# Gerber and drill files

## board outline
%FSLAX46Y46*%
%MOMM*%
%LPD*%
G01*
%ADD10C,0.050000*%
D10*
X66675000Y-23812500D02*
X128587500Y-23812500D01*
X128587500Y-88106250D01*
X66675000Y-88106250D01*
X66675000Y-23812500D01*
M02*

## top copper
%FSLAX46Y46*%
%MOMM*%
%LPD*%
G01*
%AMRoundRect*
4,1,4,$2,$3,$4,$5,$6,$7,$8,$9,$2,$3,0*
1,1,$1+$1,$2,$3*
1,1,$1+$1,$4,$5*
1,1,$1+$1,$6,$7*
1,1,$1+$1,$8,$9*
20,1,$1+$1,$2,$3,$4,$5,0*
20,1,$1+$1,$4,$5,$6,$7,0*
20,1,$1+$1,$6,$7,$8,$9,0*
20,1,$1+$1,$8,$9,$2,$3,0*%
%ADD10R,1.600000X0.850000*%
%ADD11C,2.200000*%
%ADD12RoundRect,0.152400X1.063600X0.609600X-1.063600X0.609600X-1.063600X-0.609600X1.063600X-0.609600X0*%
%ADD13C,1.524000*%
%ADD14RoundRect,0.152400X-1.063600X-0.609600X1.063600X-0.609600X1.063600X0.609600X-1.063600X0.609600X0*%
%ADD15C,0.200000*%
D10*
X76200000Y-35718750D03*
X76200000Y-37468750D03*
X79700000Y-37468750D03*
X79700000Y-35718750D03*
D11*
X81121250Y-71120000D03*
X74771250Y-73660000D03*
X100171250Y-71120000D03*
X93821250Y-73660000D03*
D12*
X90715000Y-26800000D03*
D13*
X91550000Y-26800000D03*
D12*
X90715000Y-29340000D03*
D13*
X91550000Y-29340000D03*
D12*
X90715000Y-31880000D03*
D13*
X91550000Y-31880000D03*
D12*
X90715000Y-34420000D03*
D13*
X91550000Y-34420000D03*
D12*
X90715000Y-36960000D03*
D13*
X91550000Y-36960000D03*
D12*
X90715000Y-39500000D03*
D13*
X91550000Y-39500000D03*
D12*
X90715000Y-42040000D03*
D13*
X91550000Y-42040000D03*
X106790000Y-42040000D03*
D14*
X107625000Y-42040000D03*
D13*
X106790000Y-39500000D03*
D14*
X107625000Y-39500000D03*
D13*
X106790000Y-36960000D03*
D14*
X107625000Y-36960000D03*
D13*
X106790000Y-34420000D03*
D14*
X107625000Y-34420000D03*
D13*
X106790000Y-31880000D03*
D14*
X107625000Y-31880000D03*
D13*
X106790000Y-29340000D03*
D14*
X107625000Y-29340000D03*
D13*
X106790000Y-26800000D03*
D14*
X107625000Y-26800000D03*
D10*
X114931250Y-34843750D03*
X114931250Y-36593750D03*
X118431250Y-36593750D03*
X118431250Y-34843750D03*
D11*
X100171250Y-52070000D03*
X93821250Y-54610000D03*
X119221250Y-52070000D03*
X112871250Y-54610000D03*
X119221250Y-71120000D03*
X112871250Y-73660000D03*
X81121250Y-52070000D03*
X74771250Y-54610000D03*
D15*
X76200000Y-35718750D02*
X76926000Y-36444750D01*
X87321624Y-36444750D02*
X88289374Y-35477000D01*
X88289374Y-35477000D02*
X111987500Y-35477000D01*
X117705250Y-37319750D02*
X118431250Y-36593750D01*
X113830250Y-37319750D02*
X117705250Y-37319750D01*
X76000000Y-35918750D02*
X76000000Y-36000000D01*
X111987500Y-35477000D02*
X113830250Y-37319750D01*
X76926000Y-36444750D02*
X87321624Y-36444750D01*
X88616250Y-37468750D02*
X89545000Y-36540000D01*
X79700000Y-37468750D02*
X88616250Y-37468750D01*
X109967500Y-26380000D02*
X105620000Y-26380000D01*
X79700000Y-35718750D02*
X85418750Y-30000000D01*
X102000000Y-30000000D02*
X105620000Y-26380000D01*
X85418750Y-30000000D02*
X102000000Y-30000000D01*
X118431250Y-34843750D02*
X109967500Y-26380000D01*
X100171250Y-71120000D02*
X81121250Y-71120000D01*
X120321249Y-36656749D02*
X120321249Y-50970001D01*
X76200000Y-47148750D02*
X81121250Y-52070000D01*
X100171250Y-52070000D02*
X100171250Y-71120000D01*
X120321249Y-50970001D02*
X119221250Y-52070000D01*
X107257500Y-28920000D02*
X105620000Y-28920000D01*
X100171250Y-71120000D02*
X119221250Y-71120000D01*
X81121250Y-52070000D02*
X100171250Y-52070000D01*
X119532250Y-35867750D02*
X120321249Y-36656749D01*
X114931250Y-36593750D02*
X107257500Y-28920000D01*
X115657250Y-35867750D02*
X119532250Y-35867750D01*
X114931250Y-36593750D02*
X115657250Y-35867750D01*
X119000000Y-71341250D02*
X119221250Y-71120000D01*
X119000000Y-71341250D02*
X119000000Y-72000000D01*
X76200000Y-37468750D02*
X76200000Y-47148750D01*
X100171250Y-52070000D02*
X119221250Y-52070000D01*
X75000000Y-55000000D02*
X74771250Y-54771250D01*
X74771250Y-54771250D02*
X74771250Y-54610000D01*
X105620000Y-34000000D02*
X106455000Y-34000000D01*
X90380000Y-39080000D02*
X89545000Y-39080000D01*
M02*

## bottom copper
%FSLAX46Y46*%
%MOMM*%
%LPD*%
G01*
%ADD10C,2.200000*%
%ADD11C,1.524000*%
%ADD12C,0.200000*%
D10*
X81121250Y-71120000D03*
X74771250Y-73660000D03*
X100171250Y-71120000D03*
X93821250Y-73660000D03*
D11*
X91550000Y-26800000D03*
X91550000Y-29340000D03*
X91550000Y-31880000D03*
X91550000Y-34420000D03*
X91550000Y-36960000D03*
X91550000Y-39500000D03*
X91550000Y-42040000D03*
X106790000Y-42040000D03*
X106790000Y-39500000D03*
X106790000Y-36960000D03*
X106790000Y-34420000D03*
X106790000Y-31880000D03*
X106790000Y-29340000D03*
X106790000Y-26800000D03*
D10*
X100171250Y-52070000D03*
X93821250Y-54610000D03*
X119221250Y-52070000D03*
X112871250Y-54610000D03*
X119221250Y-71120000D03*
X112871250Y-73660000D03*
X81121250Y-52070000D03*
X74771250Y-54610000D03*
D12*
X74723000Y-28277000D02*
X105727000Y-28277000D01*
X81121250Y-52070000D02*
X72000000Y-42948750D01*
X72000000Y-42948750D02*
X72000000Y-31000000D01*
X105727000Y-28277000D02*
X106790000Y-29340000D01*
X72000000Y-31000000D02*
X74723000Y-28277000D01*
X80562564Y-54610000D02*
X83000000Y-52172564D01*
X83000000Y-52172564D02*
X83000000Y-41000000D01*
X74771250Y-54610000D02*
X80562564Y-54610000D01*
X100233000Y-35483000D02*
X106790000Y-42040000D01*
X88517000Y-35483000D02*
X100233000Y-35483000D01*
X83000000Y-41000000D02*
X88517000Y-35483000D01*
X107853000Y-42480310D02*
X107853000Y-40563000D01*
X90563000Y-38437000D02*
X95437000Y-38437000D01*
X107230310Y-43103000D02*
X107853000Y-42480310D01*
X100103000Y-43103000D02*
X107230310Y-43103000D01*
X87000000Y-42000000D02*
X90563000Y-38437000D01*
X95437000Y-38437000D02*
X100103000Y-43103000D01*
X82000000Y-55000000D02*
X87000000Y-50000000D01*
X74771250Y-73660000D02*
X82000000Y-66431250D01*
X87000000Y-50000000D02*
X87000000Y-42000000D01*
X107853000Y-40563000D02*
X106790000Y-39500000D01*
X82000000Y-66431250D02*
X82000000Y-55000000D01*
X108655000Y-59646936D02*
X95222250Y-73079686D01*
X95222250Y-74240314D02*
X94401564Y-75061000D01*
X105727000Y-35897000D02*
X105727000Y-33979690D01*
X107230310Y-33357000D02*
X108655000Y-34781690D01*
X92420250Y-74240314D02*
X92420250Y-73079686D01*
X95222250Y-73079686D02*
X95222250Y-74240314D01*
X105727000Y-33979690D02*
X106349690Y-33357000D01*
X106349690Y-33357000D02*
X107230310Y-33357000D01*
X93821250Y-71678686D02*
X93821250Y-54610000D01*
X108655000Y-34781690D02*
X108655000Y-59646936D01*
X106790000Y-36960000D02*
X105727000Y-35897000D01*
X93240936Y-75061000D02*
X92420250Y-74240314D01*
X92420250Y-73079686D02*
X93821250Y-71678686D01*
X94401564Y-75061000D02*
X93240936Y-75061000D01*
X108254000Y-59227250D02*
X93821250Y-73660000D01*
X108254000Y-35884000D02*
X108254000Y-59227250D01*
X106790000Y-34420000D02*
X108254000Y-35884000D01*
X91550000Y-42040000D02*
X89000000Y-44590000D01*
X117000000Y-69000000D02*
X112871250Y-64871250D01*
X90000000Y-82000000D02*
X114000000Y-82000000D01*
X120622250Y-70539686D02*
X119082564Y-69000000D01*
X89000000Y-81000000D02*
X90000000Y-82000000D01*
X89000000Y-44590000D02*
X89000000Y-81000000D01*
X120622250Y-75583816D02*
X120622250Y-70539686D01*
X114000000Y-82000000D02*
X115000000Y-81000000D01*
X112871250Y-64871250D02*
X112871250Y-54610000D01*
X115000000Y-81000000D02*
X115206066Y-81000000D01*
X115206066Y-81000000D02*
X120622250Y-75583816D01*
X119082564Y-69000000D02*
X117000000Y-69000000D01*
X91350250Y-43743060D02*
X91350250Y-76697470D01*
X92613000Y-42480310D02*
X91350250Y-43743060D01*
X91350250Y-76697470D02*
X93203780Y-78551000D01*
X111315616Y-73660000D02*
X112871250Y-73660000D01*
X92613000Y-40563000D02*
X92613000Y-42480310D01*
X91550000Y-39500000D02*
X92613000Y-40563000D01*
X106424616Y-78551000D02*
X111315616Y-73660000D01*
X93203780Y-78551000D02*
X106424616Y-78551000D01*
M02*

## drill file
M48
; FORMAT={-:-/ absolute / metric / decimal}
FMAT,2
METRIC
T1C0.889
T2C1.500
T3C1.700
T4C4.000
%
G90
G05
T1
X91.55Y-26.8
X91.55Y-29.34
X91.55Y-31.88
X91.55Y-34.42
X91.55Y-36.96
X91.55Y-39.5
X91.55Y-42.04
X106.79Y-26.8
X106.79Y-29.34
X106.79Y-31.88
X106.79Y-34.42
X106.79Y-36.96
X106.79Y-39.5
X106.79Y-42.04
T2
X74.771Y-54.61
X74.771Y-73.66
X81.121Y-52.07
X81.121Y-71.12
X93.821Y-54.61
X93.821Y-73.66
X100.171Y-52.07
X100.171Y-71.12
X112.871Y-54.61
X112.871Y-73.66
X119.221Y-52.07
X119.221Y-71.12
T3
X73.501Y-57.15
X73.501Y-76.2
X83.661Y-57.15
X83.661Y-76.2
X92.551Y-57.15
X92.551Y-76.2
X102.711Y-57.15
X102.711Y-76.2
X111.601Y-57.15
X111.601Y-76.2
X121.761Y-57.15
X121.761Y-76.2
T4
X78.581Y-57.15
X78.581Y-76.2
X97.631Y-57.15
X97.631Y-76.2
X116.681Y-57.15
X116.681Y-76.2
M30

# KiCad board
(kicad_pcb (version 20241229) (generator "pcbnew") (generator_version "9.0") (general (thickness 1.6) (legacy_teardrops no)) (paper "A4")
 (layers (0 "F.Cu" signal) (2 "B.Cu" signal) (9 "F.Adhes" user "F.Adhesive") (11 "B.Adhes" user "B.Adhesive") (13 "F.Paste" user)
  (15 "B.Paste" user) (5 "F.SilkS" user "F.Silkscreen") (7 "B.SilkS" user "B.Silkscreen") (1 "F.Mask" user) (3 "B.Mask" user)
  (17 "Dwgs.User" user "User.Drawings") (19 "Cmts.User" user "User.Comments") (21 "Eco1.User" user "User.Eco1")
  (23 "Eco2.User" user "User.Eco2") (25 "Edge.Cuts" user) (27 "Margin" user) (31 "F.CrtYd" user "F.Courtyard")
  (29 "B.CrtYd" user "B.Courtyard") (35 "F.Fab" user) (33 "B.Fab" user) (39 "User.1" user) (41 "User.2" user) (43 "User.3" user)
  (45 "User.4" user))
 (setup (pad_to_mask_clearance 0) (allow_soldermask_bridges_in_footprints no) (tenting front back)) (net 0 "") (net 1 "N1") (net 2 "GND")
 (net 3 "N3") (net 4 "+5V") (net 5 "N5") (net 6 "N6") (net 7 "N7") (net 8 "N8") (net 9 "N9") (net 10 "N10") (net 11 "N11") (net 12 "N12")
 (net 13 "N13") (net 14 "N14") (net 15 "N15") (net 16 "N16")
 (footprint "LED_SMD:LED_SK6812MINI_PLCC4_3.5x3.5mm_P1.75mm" (layer "F.Cu") (at 77.95 36.59375)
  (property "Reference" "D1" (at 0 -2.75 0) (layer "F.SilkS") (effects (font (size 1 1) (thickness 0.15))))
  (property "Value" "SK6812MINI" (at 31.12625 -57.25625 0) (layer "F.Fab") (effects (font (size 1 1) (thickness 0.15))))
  (pad "1" smd rect (at -1.75 -0.875) (size 1.6 0.85) (layers "F.Cu" "F.Mask" "F.Paste") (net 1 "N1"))
  (pad "2" smd rect (at -1.75 0.875) (size 1.6 0.85) (layers "F.Cu" "F.Mask" "F.Paste") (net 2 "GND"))
  (pad "3" smd rect (at 1.75 0.875) (size 1.6 0.85) (layers "F.Cu" "F.Mask" "F.Paste") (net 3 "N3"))
  (pad "4" smd rect (at 1.75 -0.875) (size 1.6 0.85) (layers "F.Cu" "F.Mask" "F.Paste") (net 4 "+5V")))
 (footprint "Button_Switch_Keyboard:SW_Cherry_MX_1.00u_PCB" (layer "F.Cu") (at 81.12125 71.12)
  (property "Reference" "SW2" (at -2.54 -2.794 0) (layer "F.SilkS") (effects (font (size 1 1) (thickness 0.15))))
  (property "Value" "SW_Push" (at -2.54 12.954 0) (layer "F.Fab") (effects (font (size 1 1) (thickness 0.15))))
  (pad "" np_thru_hole circle (at -7.62 5.08) (size 1.7 1.7) (drill 1.7) (layers "*.Cu" "*.Mask"))
  (pad "" np_thru_hole circle (at -2.54 5.08) (size 4 4) (drill 4) (layers "*.Cu" "*.Mask"))
  (pad "" np_thru_hole circle (at 2.54 5.08) (size 1.7 1.7) (drill 1.7) (layers "*.Cu" "*.Mask"))
  (pad "1" thru_hole circle (at 0 0) (size 2.2 2.2) (drill 1.5) (layers "*.Cu" "*.Mask") (remove_unused_layers no) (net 2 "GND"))
  (pad "2" thru_hole circle (at -6.35 2.54) (size 2.2 2.2) (drill 1.5) (layers "*.Cu" "*.Mask") (remove_unused_layers no) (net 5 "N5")))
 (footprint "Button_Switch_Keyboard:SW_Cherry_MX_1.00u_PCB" (layer "F.Cu") (at 100.17125 71.12)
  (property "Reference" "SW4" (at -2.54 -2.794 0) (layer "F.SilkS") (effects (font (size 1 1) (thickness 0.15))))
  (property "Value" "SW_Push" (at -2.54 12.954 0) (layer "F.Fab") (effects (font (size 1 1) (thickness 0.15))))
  (pad "" np_thru_hole circle (at -7.62 5.08) (size 1.7 1.7) (drill 1.7) (layers "*.Cu" "*.Mask"))
  (pad "" np_thru_hole circle (at -2.54 5.08) (size 4 4) (drill 4) (layers "*.Cu" "*.Mask"))
  (pad "" np_thru_hole circle (at 2.54 5.08) (size 1.7 1.7) (drill 1.7) (layers "*.Cu" "*.Mask"))
  (pad "1" thru_hole circle (at 0 0) (size 2.2 2.2) (drill 1.5) (layers "*.Cu" "*.Mask") (remove_unused_layers no) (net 2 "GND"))
  (pad "2" thru_hole circle (at -6.35 2.54) (size 2.2 2.2) (drill 1.5) (layers "*.Cu" "*.Mask") (remove_unused_layers no) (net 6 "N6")))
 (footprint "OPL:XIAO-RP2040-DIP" (layer "F.Cu") (at 99.17 34.42)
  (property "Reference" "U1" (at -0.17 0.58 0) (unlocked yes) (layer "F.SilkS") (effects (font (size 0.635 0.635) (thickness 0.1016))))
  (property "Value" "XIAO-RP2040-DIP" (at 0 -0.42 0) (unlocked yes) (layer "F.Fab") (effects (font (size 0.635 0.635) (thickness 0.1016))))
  (pad "1" smd roundrect (at -8.455 -7.62 180) (size 2.432 1.524) (layers "F.Cu" "F.Mask") (roundrect_rratio 0.1) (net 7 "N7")
   (thermal_bridge_angle 45))
  (pad "1" thru_hole circle (at -7.62 -7.62 180) (size 1.524 1.524) (drill 0.889) (layers "*.Cu" "*.Mask") (remove_unused_layers no)
   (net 7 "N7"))
  (pad "2" smd roundrect (at -8.455 -5.08 180) (size 2.432 1.524) (layers "F.Cu" "F.Mask") (roundrect_rratio 0.1) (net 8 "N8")
   (thermal_bridge_angle 45))
  (pad "2" thru_hole circle (at -7.62 -5.08 180) (size 1.524 1.524) (drill 0.889) (layers "*.Cu" "*.Mask") (remove_unused_layers no)
   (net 8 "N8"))
  (pad "3" smd roundrect (at -8.455 -2.54 180) (size 2.432 1.524) (layers "F.Cu" "F.Mask") (roundrect_rratio 0.1) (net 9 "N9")
   (thermal_bridge_angle 45))
  (pad "3" thru_hole circle (at -7.62 -2.54 180) (size 1.524 1.524) (drill 0.889) (layers "*.Cu" "*.Mask") (remove_unused_layers no)
   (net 9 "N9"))
  (pad "4" smd roundrect (at -8.455 0 180) (size 2.432 1.524) (layers "F.Cu" "F.Mask") (roundrect_rratio 0.1) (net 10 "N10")
   (thermal_bridge_angle 45))
  (pad "4" thru_hole circle (at -7.62 0 180) (size 1.524 1.524) (drill 0.889) (layers "*.Cu" "*.Mask") (remove_unused_layers no)
   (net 10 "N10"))
  (pad "5" smd roundrect (at -8.455 2.54 180) (size 2.432 1.524) (layers "F.Cu" "F.Mask") (roundrect_rratio 0.1) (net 3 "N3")
   (thermal_bridge_angle 45))
  (pad "5" thru_hole circle (at -7.62 2.54 180) (size 1.524 1.524) (drill 0.889) (layers "*.Cu" "*.Mask") (remove_unused_layers no)
   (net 3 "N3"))
  (pad "6" smd roundrect (at -8.455 5.08 180) (size 2.432 1.524) (layers "F.Cu" "F.Mask") (roundrect_rratio 0.1) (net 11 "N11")
   (thermal_bridge_angle 45))
  (pad "6" thru_hole circle (at -7.62 5.08 180) (size 1.524 1.524) (drill 0.889) (layers "*.Cu" "*.Mask") (remove_unused_layers no)
   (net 11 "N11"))
  (pad "7" smd roundrect (at -8.455 7.62 180) (size 2.432 1.524) (layers "F.Cu" "F.Mask") (roundrect_rratio 0.1) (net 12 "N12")
   (thermal_bridge_angle 45))
  (pad "7" thru_hole circle (at -7.62 7.62 180) (size 1.524 1.524) (drill 0.889) (layers "*.Cu" "*.Mask") (remove_unused_layers no)
   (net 12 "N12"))
  (pad "8" thru_hole circle (at 7.62 7.62) (size 1.524 1.524) (drill 0.889) (layers "*.Cu" "*.Mask") (remove_unused_layers no)
   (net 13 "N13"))
  (pad "8" smd roundrect (at 8.455 7.62) (size 2.432 1.524) (layers "F.Cu" "F.Mask") (roundrect_rratio 0.1) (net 13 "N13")
   (thermal_bridge_angle 45))
  (pad "9" thru_hole circle (at 7.62 5.08) (size 1.524 1.524) (drill 0.889) (layers "*.Cu" "*.Mask") (remove_unused_layers no) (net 5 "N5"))
  (pad "9" smd roundrect (at 8.455 5.08) (size 2.432 1.524) (layers "F.Cu" "F.Mask") (roundrect_rratio 0.1) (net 5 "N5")
   (thermal_bridge_angle 45))
  (pad "10" thru_hole circle (at 7.62 2.54) (size 1.524 1.524) (drill 0.889) (layers "*.Cu" "*.Mask") (remove_unused_layers no)
   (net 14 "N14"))
  (pad "10" smd roundrect (at 8.455 2.54) (size 2.432 1.524) (layers "F.Cu" "F.Mask") (roundrect_rratio 0.1) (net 14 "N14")
   (thermal_bridge_angle 45))
  (pad "11" thru_hole circle (at 7.62 0) (size 1.524 1.524) (drill 0.889) (layers "*.Cu" "*.Mask") (remove_unused_layers no) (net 6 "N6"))
  (pad "11" smd roundrect (at 8.455 0) (size 2.432 1.524) (layers "F.Cu" "F.Mask") (roundrect_rratio 0.1) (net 6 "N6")
   (thermal_bridge_angle 45))
  (pad "12" thru_hole circle (at 7.62 -2.54) (size 1.524 1.524) (drill 0.889) (layers "*.Cu" "*.Mask") (remove_unused_layers no)
   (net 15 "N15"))
  (pad "12" smd roundrect (at 8.455 -2.54) (size 2.432 1.524) (layers "F.Cu" "F.Mask") (roundrect_rratio 0.1) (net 15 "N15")
   (thermal_bridge_angle 45))
  (pad "13" thru_hole circle (at 7.62 -5.08) (size 1.524 1.524) (drill 0.889) (layers "*.Cu" "*.Mask") (remove_unused_layers no)
   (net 2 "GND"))
  (pad "13" smd roundrect (at 8.455 -5.08) (size 2.432 1.524) (layers "F.Cu" "F.Mask") (roundrect_rratio 0.1) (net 2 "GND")
   (thermal_bridge_angle 45))
  (pad "14" thru_hole circle (at 7.62 -7.62) (size 1.524 1.524) (drill 0.889) (layers "*.Cu" "*.Mask") (remove_unused_layers no)
   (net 4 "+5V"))
  (pad "14" smd roundrect (at 8.455 -7.62) (size 2.432 1.524) (layers "F.Cu" "F.Mask") (roundrect_rratio 0.1) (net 4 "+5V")
   (thermal_bridge_angle 45)))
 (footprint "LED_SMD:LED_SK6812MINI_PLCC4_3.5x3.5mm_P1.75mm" (layer "F.Cu") (at 116.68125 35.71875)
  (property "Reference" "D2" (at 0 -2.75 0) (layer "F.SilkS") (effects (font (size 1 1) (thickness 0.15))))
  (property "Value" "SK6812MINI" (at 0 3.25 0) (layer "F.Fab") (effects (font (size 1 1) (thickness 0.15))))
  (pad "1" smd rect (at -1.75 -0.875) (size 1.6 0.85) (layers "F.Cu" "F.Mask" "F.Paste") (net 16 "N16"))
  (pad "2" smd rect (at -1.75 0.875) (size 1.6 0.85) (layers "F.Cu" "F.Mask" "F.Paste") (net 2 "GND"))
  (pad "3" smd rect (at 1.75 0.875) (size 1.6 0.85) (layers "F.Cu" "F.Mask" "F.Paste") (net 1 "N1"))
  (pad "4" smd rect (at 1.75 -0.875) (size 1.6 0.85) (layers "F.Cu" "F.Mask" "F.Paste") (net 4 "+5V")))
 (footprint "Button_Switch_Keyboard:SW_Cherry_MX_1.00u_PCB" (layer "F.Cu") (at 100.17125 52.07)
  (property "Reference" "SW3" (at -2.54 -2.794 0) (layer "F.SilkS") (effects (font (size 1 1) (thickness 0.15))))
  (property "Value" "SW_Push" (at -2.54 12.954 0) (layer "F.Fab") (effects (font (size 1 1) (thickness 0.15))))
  (pad "" np_thru_hole circle (at -7.62 5.08) (size 1.7 1.7) (drill 1.7) (layers "*.Cu" "*.Mask"))
  (pad "" np_thru_hole circle (at -2.54 5.08) (size 4 4) (drill 4) (layers "*.Cu" "*.Mask"))
  (pad "" np_thru_hole circle (at 2.54 5.08) (size 1.7 1.7) (drill 1.7) (layers "*.Cu" "*.Mask"))
  (pad "1" thru_hole circle (at 0 0) (size 2.2 2.2) (drill 1.5) (layers "*.Cu" "*.Mask") (remove_unused_layers no) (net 2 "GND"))
  (pad "2" thru_hole circle (at -6.35 2.54) (size 2.2 2.2) (drill 1.5) (layers "*.Cu" "*.Mask") (remove_unused_layers no) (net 14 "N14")))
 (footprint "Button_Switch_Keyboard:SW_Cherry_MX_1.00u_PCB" (layer "F.Cu") (at 119.22125 52.07)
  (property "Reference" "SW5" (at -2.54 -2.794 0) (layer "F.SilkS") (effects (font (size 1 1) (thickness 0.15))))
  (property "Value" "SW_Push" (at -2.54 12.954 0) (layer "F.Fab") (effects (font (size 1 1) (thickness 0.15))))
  (pad "" np_thru_hole circle (at -7.62 5.08) (size 1.7 1.7) (drill 1.7) (layers "*.Cu" "*.Mask"))
  (pad "" np_thru_hole circle (at -2.54 5.08) (size 4 4) (drill 4) (layers "*.Cu" "*.Mask"))
  (pad "" np_thru_hole circle (at 2.54 5.08) (size 1.7 1.7) (drill 1.7) (layers "*.Cu" "*.Mask"))
  (pad "1" thru_hole circle (at 0 0) (size 2.2 2.2) (drill 1.5) (layers "*.Cu" "*.Mask") (remove_unused_layers no) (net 2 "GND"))
  (pad "2" thru_hole circle (at -6.35 2.54) (size 2.2 2.2) (drill 1.5) (layers "*.Cu" "*.Mask") (remove_unused_layers no) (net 12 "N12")))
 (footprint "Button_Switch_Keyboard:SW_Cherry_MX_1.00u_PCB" (layer "F.Cu") (at 119.22125 71.12)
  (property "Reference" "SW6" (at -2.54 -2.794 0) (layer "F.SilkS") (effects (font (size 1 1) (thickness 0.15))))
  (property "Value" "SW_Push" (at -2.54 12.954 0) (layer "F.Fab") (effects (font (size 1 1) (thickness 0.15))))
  (pad "" np_thru_hole circle (at -7.62 5.08) (size 1.7 1.7) (drill 1.7) (layers "*.Cu" "*.Mask"))
  (pad "" np_thru_hole circle (at -2.54 5.08) (size 4 4) (drill 4) (layers "*.Cu" "*.Mask"))
  (pad "" np_thru_hole circle (at 2.54 5.08) (size 1.7 1.7) (drill 1.7) (layers "*.Cu" "*.Mask"))
  (pad "1" thru_hole circle (at 0 0) (size 2.2 2.2) (drill 1.5) (layers "*.Cu" "*.Mask") (remove_unused_layers no) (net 2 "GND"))
  (pad "2" thru_hole circle (at -6.35 2.54) (size 2.2 2.2) (drill 1.5) (layers "*.Cu" "*.Mask") (remove_unused_layers no) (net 11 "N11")))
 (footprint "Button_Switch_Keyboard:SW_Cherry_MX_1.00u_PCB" (layer "F.Cu") (at 81.12125 52.07)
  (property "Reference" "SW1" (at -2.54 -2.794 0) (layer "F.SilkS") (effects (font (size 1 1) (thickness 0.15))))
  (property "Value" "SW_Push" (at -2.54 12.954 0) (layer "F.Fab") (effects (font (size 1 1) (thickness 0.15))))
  (pad "" np_thru_hole circle (at -7.62 5.08) (size 1.7 1.7) (drill 1.7) (layers "*.Cu" "*.Mask"))
  (pad "" np_thru_hole circle (at -2.54 5.08) (size 4 4) (drill 4) (layers "*.Cu" "*.Mask"))
  (pad "" np_thru_hole circle (at 2.54 5.08) (size 1.7 1.7) (drill 1.7) (layers "*.Cu" "*.Mask"))
  (pad "1" thru_hole circle (at 0 0) (size 2.2 2.2) (drill 1.5) (layers "*.Cu" "*.Mask") (remove_unused_layers no) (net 2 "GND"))
  (pad "2" thru_hole circle (at -6.35 2.54) (size 2.2 2.2) (drill 1.5) (layers "*.Cu" "*.Mask") (remove_unused_layers no) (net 13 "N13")))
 (gr_rect (start 66.675 23.8125) (end 128.5875 88.10625) (stroke (width 0.05) (type default)) (fill no) (layer "Edge.Cuts"))
 (segment (start 76.2 35.71875) (end 76.926 36.44475) (width 0.2) (layer "F.Cu") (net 1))
 (segment (start 87.321624 36.44475) (end 88.289374 35.477) (width 0.2) (layer "F.Cu") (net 1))
 (segment (start 88.289374 35.477) (end 111.9875 35.477) (width 0.2) (layer "F.Cu") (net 1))
 (segment (start 117.70525 37.31975) (end 118.43125 36.59375) (width 0.2) (layer "F.Cu") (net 1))
 (segment (start 113.83025 37.31975) (end 117.70525 37.31975) (width 0.2) (layer "F.Cu") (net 1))
 (segment (start 76 35.91875) (end 76 36) (width 0.2) (layer "F.Cu") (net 1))
 (segment (start 111.9875 35.477) (end 113.83025 37.31975) (width 0.2) (layer "F.Cu") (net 1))
 (segment (start 76.926 36.44475) (end 87.321624 36.44475) (width 0.2) (layer "F.Cu") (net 1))
 (segment (start 88.61625 37.46875) (end 89.545 36.54) (width 0.2) (layer "F.Cu") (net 3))
 (segment (start 79.7 37.46875) (end 88.61625 37.46875) (width 0.2) (layer "F.Cu") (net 3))
 (segment (start 109.9675 26.38) (end 105.62 26.38) (width 0.2) (layer "F.Cu") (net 4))
 (segment (start 79.7 35.71875) (end 85.41875 30) (width 0.2) (layer "F.Cu") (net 4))
 (segment (start 102 30) (end 105.62 26.38) (width 0.2) (layer "F.Cu") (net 4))
 (segment (start 85.41875 30) (end 102 30) (width 0.2) (layer "F.Cu") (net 4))
 (segment (start 118.43125 34.84375) (end 109.9675 26.38) (width 0.2) (layer "F.Cu") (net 4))
 (segment (start 100.17125 71.12) (end 81.12125 71.12) (width 0.2) (layer "F.Cu") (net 2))
 (segment (start 120.321249 36.656749) (end 120.321249 50.970001) (width 0.2) (layer "F.Cu") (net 2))
 (segment (start 76.2 47.14875) (end 81.12125 52.07) (width 0.2) (layer "F.Cu") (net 2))
 (segment (start 100.17125 52.07) (end 100.17125 71.12) (width 0.2) (layer "F.Cu") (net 2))
 (segment (start 120.321249 50.970001) (end 119.22125 52.07) (width 0.2) (layer "F.Cu") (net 2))
 (segment (start 107.2575 28.92) (end 105.62 28.92) (width 0.2) (layer "F.Cu") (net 2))
 (segment (start 100.17125 71.12) (end 119.22125 71.12) (width 0.2) (layer "F.Cu") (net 2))
 (segment (start 81.12125 52.07) (end 100.17125 52.07) (width 0.2) (layer "F.Cu") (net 2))
 (segment (start 119.53225 35.86775) (end 120.321249 36.656749) (width 0.2) (layer "F.Cu") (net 2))
 (segment (start 114.93125 36.59375) (end 107.2575 28.92) (width 0.2) (layer "F.Cu") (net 2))
 (segment (start 115.65725 35.86775) (end 119.53225 35.86775) (width 0.2) (layer "F.Cu") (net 2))
 (segment (start 114.93125 36.59375) (end 115.65725 35.86775) (width 0.2) (layer "F.Cu") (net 2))
 (segment (start 119 71.34125) (end 119.22125 71.12) (width 0.2) (layer "F.Cu") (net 2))
 (segment (start 119 71.34125) (end 119 72) (width 0.2) (layer "F.Cu") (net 2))
 (segment (start 76.2 37.46875) (end 76.2 47.14875) (width 0.2) (layer "F.Cu") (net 2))
 (segment (start 100.17125 52.07) (end 119.22125 52.07) (width 0.2) (layer "F.Cu") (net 2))
 (segment (start 74.723 28.277) (end 105.727 28.277) (width 0.2) (layer "B.Cu") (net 2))
 (segment (start 81.12125 52.07) (end 72 42.94875) (width 0.2) (layer "B.Cu") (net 2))
 (segment (start 72 42.94875) (end 72 31) (width 0.2) (layer "B.Cu") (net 2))
 (segment (start 105.727 28.277) (end 106.79 29.34) (width 0.2) (layer "B.Cu") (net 2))
 (segment (start 72 31) (end 74.723 28.277) (width 0.2) (layer "B.Cu") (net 2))
 (segment (start 75 55) (end 74.77125 54.77125) (width 0.2) (layer "F.Cu") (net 13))
 (segment (start 74.77125 54.77125) (end 74.77125 54.61) (width 0.2) (layer "F.Cu") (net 13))
 (segment (start 80.562564 54.61) (end 83 52.172564) (width 0.2) (layer "B.Cu") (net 13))
 (segment (start 83 52.172564) (end 83 41) (width 0.2) (layer "B.Cu") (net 13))
 (segment (start 74.77125 54.61) (end 80.562564 54.61) (width 0.2) (layer "B.Cu") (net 13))
 (segment (start 100.233 35.483) (end 106.79 42.04) (width 0.2) (layer "B.Cu") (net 13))
 (segment (start 88.517 35.483) (end 100.233 35.483) (width 0.2) (layer "B.Cu") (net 13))
 (segment (start 83 41) (end 88.517 35.483) (width 0.2) (layer "B.Cu") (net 13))
 (segment (start 107.853 42.48031) (end 107.853 40.563) (width 0.2) (layer "B.Cu") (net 5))
 (segment (start 90.563 38.437) (end 95.437 38.437) (width 0.2) (layer "B.Cu") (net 5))
 (segment (start 107.23031 43.103) (end 107.853 42.48031) (width 0.2) (layer "B.Cu") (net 5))
 (segment (start 100.103 43.103) (end 107.23031 43.103) (width 0.2) (layer "B.Cu") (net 5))
 (segment (start 87 42) (end 90.563 38.437) (width 0.2) (layer "B.Cu") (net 5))
 (segment (start 95.437 38.437) (end 100.103 43.103) (width 0.2) (layer "B.Cu") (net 5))
 (segment (start 82 55) (end 87 50) (width 0.2) (layer "B.Cu") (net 5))
 (segment (start 74.77125 73.66) (end 82 66.43125) (width 0.2) (layer "B.Cu") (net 5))
 (segment (start 87 50) (end 87 42) (width 0.2) (layer "B.Cu") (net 5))
 (segment (start 107.853 40.563) (end 106.79 39.5) (width 0.2) (layer "B.Cu") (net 5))
 (segment (start 82 66.43125) (end 82 55) (width 0.2) (layer "B.Cu") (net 5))
 (segment (start 108.655 59.646936) (end 95.22225 73.079686) (width 0.2) (layer "B.Cu") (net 14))
 (segment (start 95.22225 74.240314) (end 94.401564 75.061) (width 0.2) (layer "B.Cu") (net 14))
 (segment (start 105.727 35.897) (end 105.727 33.97969) (width 0.2) (layer "B.Cu") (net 14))
 (segment (start 107.23031 33.357) (end 108.655 34.78169) (width 0.2) (layer "B.Cu") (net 14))
 (segment (start 92.42025 74.240314) (end 92.42025 73.079686) (width 0.2) (layer "B.Cu") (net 14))
 (segment (start 95.22225 73.079686) (end 95.22225 74.240314) (width 0.2) (layer "B.Cu") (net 14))
 (segment (start 105.727 33.97969) (end 106.34969 33.357) (width 0.2) (layer "B.Cu") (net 14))
 (segment (start 106.34969 33.357) (end 107.23031 33.357) (width 0.2) (layer "B.Cu") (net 14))
 (segment (start 93.82125 71.678686) (end 93.82125 54.61) (width 0.2) (layer "B.Cu") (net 14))
 (segment (start 108.655 34.78169) (end 108.655 59.646936) (width 0.2) (layer "B.Cu") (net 14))
 (segment (start 106.79 36.96) (end 105.727 35.897) (width 0.2) (layer "B.Cu") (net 14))
 (segment (start 93.240936 75.061) (end 92.42025 74.240314) (width 0.2) (layer "B.Cu") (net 14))
 (segment (start 92.42025 73.079686) (end 93.82125 71.678686) (width 0.2) (layer "B.Cu") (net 14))
 (segment (start 94.401564 75.061) (end 93.240936 75.061) (width 0.2) (layer "B.Cu") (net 14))
 (segment (start 105.62 34) (end 106.455 34) (width 0.2) (layer "F.Cu") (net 6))
 (segment (start 108.254 59.22725) (end 93.82125 73.66) (width 0.2) (layer "B.Cu") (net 6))
 (segment (start 108.254 35.884) (end 108.254 59.22725) (width 0.2) (layer "B.Cu") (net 6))
 (segment (start 106.79 34.42) (end 108.254 35.884) (width 0.2) (layer "B.Cu") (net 6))
 (segment (start 91.55 42.04) (end 89 44.59) (width 0.2) (layer "B.Cu") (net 12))
 (segment (start 117 69) (end 112.87125 64.87125) (width 0.2) (layer "B.Cu") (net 12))
 (segment (start 90 82) (end 114 82) (width 0.2) (layer "B.Cu") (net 12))
 (segment (start 120.62225 70.539686) (end 119.082564 69) (width 0.2) (layer "B.Cu") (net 12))
 (segment (start 89 81) (end 90 82) (width 0.2) (layer "B.Cu") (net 12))
 (segment (start 89 44.59) (end 89 81) (width 0.2) (layer "B.Cu") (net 12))
 (segment (start 120.62225 75.583816) (end 120.62225 70.539686) (width 0.2) (layer "B.Cu") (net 12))
 (segment (start 114 82) (end 115 81) (width 0.2) (layer "B.Cu") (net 12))
 (segment (start 112.87125 64.87125) (end 112.87125 54.61) (width 0.2) (layer "B.Cu") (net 12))
 (segment (start 115 81) (end 115.206066 81) (width 0.2) (layer "B.Cu") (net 12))
 (segment (start 115.206066 81) (end 120.62225 75.583816) (width 0.2) (layer "B.Cu") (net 12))
 (segment (start 119.082564 69) (end 117 69) (width 0.2) (layer "B.Cu") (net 12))
 (segment (start 90.38 39.08) (end 89.545 39.08) (width 0.2) (layer "F.Cu") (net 11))
 (segment (start 91.35025 43.74306) (end 91.35025 76.69747) (width 0.2) (layer "B.Cu") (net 11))
 (segment (start 92.613 42.48031) (end 91.35025 43.74306) (width 0.2) (layer "B.Cu") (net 11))
 (segment (start 91.35025 76.69747) (end 93.20378 78.551) (width 0.2) (layer "B.Cu") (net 11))
 (segment (start 111.315616 73.66) (end 112.87125 73.66) (width 0.2) (layer "B.Cu") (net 11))
 (segment (start 92.613 40.563) (end 92.613 42.48031) (width 0.2) (layer "B.Cu") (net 11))
 (segment (start 91.55 39.5) (end 92.613 40.563) (width 0.2) (layer "B.Cu") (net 11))
 (segment (start 106.424616 78.551) (end 111.315616 73.66) (width 0.2) (layer "B.Cu") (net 11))
 (segment (start 93.20378 78.551) (end 106.424616 78.551) (width 0.2) (layer "B.Cu") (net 11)))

